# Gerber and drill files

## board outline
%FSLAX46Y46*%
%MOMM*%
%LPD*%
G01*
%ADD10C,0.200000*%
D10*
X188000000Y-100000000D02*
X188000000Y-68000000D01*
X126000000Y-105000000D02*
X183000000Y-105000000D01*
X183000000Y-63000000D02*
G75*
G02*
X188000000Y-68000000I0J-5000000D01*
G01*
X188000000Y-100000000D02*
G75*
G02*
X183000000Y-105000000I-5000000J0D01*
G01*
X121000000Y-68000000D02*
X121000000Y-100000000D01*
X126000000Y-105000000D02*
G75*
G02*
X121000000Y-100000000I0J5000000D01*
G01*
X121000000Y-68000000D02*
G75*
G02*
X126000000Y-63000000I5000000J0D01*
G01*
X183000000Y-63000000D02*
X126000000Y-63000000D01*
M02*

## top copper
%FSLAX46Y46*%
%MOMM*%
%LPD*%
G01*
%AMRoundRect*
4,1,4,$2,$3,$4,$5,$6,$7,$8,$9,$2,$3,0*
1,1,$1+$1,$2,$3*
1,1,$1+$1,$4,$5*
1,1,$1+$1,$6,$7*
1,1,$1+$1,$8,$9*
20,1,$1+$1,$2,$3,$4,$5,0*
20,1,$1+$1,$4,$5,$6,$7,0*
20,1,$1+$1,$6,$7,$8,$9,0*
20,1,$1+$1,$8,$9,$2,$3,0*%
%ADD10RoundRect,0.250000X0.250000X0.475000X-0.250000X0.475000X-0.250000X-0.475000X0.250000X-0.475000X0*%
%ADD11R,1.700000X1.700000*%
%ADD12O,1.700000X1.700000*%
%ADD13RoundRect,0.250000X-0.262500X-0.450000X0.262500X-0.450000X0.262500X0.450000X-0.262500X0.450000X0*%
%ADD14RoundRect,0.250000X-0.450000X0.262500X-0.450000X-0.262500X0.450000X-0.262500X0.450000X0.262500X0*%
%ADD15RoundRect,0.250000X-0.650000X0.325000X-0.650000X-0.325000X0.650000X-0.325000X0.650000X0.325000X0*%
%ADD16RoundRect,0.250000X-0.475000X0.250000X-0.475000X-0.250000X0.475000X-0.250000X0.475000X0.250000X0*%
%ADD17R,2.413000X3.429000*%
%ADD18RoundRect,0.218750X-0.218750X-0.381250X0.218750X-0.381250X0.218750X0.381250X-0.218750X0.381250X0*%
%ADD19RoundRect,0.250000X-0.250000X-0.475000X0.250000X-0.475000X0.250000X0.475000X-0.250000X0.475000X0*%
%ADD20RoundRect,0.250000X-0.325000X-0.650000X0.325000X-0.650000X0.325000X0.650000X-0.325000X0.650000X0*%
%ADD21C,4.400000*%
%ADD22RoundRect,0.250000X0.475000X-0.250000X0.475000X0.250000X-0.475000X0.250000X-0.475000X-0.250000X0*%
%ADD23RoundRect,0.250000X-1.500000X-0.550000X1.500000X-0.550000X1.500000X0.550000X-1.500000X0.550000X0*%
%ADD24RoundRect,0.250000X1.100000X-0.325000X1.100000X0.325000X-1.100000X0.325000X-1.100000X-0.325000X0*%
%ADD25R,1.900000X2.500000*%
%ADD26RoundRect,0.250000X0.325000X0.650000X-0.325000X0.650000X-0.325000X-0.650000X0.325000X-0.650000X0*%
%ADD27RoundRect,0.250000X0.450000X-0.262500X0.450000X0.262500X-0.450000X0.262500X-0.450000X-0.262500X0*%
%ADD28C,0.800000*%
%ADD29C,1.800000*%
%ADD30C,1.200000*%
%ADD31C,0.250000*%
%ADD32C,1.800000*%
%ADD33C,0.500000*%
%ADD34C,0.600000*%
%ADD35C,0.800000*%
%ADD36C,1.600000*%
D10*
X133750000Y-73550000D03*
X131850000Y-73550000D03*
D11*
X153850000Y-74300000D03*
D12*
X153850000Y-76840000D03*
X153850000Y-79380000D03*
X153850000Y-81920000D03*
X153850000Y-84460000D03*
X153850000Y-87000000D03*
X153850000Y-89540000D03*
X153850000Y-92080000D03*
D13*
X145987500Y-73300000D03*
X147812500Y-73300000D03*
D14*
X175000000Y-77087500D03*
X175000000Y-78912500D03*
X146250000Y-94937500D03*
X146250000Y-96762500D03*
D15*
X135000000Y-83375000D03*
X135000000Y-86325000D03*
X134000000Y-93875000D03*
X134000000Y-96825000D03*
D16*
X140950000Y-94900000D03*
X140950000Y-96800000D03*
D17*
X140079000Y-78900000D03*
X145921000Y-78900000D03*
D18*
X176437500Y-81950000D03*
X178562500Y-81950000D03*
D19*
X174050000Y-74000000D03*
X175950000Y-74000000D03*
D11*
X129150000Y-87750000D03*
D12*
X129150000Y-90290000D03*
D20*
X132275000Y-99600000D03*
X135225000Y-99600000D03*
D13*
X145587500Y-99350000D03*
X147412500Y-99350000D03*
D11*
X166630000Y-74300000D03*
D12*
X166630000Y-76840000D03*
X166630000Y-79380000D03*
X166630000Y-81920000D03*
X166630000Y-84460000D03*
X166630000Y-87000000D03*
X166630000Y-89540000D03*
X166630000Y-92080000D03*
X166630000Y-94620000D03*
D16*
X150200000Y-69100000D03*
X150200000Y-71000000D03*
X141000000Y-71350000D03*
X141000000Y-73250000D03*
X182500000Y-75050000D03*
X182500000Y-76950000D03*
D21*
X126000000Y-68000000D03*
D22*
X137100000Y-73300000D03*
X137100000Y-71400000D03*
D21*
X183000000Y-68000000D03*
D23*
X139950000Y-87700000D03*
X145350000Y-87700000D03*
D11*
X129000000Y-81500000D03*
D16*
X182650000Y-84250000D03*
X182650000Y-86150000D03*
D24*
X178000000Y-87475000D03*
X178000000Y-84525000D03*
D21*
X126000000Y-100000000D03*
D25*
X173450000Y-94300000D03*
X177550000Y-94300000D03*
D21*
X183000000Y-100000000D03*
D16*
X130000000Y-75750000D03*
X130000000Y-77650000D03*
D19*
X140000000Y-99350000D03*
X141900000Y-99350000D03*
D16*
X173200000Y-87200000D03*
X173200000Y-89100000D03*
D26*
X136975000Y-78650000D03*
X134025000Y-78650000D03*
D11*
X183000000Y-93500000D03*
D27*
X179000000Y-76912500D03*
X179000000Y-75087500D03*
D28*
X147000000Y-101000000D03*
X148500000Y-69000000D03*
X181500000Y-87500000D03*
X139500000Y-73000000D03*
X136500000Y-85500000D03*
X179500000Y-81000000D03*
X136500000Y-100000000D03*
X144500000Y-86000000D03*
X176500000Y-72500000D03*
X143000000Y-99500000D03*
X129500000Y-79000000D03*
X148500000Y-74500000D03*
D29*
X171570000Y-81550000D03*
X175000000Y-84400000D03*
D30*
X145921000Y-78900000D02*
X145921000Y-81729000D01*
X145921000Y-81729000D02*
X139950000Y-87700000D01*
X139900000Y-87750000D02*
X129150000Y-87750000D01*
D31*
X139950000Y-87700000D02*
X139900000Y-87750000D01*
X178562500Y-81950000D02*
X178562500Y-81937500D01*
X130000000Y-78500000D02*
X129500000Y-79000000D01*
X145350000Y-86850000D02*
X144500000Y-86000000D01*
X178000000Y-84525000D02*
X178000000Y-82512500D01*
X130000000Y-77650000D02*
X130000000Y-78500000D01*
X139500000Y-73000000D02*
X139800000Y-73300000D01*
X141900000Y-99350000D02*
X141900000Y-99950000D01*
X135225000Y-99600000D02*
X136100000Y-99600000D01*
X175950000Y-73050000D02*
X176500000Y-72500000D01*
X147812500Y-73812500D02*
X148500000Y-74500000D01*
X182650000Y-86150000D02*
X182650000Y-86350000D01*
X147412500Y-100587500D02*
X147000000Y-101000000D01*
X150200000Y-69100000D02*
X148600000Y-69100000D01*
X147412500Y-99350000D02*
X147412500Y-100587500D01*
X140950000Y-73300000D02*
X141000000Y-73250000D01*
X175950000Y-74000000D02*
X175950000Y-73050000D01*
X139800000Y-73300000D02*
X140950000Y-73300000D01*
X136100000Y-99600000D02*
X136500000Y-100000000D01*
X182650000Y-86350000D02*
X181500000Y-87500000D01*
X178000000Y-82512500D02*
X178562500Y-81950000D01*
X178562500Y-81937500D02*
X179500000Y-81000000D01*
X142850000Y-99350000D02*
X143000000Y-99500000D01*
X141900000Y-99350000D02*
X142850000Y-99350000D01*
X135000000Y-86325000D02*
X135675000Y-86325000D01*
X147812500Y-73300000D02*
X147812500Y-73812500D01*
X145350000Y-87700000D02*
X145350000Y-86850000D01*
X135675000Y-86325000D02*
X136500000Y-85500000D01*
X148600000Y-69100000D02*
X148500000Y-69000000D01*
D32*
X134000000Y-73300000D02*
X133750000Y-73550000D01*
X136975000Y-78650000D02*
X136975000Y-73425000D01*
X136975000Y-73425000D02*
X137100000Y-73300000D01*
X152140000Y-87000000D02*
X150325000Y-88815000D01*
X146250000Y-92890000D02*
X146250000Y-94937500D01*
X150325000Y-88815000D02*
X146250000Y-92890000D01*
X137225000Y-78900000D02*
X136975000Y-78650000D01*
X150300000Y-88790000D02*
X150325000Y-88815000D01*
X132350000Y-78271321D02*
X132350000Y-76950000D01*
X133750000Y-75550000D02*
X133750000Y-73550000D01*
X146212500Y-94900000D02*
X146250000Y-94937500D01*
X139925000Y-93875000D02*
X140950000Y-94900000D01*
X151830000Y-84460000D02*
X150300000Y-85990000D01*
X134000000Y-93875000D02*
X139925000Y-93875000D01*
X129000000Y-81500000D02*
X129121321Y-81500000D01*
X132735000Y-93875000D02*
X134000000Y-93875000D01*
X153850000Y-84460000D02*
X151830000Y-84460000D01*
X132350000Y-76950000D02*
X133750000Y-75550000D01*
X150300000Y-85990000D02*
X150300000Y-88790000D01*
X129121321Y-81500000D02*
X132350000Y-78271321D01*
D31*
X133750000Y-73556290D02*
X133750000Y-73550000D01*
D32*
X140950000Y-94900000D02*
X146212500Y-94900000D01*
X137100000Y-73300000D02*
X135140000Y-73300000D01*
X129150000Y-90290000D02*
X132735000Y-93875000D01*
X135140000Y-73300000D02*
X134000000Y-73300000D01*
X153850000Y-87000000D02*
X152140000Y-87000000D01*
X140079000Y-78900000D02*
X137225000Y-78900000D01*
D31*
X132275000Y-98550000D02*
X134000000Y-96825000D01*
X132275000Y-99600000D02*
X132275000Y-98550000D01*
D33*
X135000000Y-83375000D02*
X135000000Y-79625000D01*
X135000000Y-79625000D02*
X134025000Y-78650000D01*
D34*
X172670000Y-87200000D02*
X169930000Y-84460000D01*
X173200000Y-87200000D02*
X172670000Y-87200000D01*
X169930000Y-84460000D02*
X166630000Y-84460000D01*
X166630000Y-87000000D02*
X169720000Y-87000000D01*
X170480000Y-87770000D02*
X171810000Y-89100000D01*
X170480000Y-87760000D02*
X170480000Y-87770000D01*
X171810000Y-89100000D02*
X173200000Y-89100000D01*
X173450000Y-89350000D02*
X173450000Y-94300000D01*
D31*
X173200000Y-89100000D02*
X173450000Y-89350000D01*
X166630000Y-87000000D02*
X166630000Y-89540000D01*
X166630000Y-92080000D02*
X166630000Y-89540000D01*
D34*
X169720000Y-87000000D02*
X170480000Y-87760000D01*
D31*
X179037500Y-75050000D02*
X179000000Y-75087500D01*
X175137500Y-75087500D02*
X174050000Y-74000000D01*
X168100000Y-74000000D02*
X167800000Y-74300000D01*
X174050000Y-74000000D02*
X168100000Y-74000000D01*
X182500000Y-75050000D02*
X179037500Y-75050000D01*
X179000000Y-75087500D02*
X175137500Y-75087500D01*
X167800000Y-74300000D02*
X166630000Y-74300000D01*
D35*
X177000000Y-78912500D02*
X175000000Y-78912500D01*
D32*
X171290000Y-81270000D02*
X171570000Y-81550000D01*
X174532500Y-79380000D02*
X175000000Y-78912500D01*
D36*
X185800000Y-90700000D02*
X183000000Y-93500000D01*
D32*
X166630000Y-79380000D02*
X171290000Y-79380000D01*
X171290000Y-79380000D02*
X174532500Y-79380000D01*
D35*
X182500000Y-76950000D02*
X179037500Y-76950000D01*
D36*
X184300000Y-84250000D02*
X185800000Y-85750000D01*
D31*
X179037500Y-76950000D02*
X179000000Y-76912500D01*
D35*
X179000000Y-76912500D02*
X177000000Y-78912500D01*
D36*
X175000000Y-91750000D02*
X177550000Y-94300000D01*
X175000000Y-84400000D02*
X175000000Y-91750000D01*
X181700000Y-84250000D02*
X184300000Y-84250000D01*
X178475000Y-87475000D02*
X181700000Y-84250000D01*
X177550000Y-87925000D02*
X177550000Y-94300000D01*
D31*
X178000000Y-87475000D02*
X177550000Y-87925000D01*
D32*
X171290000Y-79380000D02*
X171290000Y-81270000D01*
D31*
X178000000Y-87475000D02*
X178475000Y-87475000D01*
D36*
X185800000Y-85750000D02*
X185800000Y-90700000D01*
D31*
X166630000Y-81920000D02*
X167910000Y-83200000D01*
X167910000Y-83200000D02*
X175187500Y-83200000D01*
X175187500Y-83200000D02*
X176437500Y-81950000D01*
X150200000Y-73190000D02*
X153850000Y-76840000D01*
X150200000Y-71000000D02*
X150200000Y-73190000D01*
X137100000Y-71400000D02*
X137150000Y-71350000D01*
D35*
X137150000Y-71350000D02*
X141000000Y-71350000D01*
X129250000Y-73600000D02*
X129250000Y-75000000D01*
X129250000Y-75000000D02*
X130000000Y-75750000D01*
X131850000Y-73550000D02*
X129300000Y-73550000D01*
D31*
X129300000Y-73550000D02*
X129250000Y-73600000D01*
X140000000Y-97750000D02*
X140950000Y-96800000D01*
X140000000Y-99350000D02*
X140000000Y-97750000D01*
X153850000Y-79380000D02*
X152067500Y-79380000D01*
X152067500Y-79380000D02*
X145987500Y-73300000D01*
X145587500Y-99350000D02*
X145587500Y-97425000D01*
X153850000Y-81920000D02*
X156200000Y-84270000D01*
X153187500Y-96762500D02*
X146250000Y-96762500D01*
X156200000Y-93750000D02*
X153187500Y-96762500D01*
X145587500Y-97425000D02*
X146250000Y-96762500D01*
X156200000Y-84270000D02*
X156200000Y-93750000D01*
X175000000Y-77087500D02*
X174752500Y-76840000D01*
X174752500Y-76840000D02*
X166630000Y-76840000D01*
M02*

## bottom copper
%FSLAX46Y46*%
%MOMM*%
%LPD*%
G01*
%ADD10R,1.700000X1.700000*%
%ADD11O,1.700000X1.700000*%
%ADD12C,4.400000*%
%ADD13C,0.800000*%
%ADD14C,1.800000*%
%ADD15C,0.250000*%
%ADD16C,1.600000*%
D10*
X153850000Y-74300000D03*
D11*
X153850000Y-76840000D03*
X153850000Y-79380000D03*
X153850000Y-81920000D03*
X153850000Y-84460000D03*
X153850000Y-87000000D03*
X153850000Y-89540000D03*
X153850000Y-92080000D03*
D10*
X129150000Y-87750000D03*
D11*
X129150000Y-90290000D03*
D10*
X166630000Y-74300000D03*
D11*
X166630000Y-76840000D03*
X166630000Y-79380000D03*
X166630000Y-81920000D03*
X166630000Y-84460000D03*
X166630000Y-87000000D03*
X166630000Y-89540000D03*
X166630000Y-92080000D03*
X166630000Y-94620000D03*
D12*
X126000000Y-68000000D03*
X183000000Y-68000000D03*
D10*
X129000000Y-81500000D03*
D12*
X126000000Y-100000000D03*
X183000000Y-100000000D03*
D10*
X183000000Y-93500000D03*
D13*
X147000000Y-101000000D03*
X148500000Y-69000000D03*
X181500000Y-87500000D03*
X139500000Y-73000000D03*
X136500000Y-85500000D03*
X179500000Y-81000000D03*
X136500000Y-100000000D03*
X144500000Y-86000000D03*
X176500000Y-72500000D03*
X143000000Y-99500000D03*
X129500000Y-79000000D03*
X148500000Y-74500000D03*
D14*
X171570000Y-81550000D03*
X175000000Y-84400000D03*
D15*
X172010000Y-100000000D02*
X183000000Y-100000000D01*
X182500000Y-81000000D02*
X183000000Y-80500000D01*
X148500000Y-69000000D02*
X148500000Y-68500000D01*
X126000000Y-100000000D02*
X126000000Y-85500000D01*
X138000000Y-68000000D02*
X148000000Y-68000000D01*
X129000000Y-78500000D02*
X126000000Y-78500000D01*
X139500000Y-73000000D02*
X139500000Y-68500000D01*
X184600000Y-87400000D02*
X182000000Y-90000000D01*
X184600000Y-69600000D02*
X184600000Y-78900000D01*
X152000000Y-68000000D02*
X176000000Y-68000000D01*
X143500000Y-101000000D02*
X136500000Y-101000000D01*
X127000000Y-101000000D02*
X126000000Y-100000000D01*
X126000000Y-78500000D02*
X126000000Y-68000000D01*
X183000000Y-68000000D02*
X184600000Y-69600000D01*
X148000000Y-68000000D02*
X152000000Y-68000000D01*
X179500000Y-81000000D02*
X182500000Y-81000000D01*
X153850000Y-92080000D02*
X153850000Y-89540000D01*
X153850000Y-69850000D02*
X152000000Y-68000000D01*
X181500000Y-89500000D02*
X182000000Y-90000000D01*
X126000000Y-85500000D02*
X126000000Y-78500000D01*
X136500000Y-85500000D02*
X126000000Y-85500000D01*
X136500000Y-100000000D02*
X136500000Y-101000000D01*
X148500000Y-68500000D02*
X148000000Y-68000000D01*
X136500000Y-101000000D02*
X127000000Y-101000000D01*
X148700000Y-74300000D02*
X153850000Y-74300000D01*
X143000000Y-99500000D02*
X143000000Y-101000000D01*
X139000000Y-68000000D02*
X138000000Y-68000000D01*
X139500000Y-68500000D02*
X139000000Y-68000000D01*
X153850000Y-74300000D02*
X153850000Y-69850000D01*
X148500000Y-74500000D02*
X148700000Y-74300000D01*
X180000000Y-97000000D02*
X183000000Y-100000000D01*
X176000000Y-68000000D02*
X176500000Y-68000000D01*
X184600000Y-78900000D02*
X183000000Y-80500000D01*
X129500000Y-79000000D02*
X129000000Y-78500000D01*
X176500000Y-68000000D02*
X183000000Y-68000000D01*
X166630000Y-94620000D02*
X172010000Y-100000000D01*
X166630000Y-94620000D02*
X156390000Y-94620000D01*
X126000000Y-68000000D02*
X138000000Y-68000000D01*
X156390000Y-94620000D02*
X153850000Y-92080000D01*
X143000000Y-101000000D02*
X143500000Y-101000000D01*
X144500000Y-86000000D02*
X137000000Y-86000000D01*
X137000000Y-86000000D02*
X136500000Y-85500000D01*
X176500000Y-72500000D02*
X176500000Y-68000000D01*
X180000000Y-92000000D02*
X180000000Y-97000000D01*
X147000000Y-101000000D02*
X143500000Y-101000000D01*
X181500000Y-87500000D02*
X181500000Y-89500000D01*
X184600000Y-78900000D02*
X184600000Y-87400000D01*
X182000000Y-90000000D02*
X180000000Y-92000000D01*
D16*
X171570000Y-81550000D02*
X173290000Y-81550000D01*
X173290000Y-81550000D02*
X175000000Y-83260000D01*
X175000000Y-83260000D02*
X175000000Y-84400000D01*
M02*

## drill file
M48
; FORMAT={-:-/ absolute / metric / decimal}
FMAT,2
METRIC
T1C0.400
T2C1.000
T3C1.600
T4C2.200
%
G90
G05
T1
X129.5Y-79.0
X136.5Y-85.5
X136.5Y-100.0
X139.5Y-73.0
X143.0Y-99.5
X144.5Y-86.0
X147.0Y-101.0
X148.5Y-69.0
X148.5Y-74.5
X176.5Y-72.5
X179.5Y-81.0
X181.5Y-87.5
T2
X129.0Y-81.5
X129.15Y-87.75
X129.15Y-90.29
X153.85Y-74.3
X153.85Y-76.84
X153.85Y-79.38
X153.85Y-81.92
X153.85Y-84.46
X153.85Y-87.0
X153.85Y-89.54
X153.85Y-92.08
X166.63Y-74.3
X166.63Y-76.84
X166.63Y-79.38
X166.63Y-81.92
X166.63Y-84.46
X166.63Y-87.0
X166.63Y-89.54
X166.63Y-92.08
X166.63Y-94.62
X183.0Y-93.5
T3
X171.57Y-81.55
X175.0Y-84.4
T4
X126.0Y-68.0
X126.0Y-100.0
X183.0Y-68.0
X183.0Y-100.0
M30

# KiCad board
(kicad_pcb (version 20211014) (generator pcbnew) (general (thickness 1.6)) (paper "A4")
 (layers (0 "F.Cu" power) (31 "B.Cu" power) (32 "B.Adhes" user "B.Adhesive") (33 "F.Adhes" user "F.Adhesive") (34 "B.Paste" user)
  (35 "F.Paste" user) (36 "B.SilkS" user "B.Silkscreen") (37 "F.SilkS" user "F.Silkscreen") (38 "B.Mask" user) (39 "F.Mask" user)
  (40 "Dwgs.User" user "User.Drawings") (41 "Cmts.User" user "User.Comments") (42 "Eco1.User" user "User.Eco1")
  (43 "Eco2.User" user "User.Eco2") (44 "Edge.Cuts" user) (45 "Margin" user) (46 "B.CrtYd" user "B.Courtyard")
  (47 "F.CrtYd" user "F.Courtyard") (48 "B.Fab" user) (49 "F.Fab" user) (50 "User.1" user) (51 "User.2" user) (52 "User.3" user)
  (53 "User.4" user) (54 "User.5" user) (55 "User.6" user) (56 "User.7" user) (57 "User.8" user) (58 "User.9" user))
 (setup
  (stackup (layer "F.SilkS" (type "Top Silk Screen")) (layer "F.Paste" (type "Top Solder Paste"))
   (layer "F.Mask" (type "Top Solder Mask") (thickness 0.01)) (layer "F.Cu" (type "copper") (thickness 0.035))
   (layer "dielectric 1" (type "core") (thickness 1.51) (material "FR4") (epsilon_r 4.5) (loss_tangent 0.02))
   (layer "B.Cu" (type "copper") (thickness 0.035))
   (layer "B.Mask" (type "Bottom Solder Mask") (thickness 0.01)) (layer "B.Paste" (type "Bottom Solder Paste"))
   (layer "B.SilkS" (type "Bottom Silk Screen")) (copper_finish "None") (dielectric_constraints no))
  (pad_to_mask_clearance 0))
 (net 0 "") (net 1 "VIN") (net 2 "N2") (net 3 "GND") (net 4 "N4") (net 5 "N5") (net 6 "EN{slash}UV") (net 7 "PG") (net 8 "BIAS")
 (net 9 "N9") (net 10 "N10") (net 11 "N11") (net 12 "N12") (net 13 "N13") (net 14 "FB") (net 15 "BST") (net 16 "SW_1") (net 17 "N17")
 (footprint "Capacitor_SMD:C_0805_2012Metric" (layer "F.Cu") (at 132.8 73.55 180)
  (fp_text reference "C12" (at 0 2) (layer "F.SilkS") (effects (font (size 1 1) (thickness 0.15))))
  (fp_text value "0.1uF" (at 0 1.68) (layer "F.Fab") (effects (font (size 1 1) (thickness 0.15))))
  (pad "1" smd roundrect (at -0.95 0 180) (size 1 1.45) (layers "F.Cu" "F.Paste" "F.Mask") (roundrect_rratio 0.25) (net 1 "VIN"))
  (pad "2" smd roundrect (at 0.95 0 180) (size 1 1.45) (layers "F.Cu" "F.Paste" "F.Mask") (roundrect_rratio 0.25) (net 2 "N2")))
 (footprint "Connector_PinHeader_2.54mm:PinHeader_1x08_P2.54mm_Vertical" (layer "F.Cu") (at 153.85 74.3)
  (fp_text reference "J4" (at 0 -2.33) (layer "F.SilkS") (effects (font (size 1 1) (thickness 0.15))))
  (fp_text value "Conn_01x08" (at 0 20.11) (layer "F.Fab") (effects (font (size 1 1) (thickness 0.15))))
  (pad "1" thru_hole rect (at 0 0) (size 1.7 1.7) (drill 1) (layers *.Cu *.Mask) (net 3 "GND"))
  (pad "2" thru_hole oval (at 0 2.54) (size 1.7 1.7) (drill 1) (layers *.Cu *.Mask) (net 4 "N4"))
  (pad "3" thru_hole oval (at 0 5.08) (size 1.7 1.7) (drill 1) (layers *.Cu *.Mask) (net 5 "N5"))
  (pad "4" thru_hole oval (at 0 7.62) (size 1.7 1.7) (drill 1) (layers *.Cu *.Mask) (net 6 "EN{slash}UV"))
  (pad "5" thru_hole oval (at 0 10.16) (size 1.7 1.7) (drill 1) (layers *.Cu *.Mask) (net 1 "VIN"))
  (pad "6" thru_hole oval (at 0 12.7) (size 1.7 1.7) (drill 1) (layers *.Cu *.Mask) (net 1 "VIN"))
  (pad "7" thru_hole oval (at 0 15.24) (size 1.7 1.7) (drill 1) (layers *.Cu *.Mask) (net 3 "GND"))
  (pad "8" thru_hole oval (at 0 17.78) (size 1.7 1.7) (drill 1) (layers *.Cu *.Mask) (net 3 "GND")))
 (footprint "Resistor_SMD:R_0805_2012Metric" (layer "F.Cu") (at 146.9 73.3)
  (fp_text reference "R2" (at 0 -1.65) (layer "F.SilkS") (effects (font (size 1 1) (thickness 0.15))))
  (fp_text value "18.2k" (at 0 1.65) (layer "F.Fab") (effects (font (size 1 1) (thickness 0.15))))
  (pad "1" smd roundrect (at -0.9125 0) (size 1.025 1.4) (layers "F.Cu" "F.Paste" "F.Mask") (roundrect_rratio 0.243902) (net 5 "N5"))
  (pad "2" smd roundrect (at 0.9125 0) (size 1.025 1.4) (layers "F.Cu" "F.Paste" "F.Mask") (roundrect_rratio 0.243902) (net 3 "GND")))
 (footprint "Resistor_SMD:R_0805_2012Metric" (layer "F.Cu") (at 175 78 -90)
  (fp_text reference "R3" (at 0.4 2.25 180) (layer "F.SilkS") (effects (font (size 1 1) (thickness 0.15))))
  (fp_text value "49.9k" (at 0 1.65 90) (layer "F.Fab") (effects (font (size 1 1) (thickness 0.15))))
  (pad "1" smd roundrect (at -0.9125 0 270) (size 1.025 1.4) (layers "F.Cu" "F.Paste" "F.Mask") (roundrect_rratio 0.243902) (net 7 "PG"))
  (pad "2" smd roundrect (at 0.9125 0 270) (size 1.025 1.4) (layers "F.Cu" "F.Paste" "F.Mask") (roundrect_rratio 0.243902) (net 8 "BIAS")))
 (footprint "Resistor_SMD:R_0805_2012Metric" (layer "F.Cu") (at 146.25 95.85 -90)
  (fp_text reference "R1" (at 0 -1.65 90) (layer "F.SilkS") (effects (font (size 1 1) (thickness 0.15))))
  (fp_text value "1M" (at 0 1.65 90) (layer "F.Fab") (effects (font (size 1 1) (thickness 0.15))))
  (pad "1" smd roundrect (at -0.9125 0 270) (size 1.025 1.4) (layers "F.Cu" "F.Paste" "F.Mask") (roundrect_rratio 0.243902) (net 1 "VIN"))
  (pad "2" smd roundrect (at 0.9125 0 270) (size 1.025 1.4) (layers "F.Cu" "F.Paste" "F.Mask") (roundrect_rratio 0.243902)
   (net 6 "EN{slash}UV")))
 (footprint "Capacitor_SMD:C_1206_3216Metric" (layer "F.Cu") (at 135 84.85 -90)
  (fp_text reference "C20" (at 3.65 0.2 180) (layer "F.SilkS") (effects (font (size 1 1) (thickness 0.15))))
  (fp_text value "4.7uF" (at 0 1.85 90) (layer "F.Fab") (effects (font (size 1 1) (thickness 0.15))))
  (pad "1" smd roundrect (at -1.475 0 270) (size 1.15 1.8) (layers "F.Cu" "F.Paste" "F.Mask") (roundrect_rratio 0.217391) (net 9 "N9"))
  (pad "2" smd roundrect (at 1.475 0 270) (size 1.15 1.8) (layers "F.Cu" "F.Paste" "F.Mask") (roundrect_rratio 0.217391) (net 3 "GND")))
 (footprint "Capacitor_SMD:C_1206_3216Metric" (layer "F.Cu") (at 134 95.35 -90)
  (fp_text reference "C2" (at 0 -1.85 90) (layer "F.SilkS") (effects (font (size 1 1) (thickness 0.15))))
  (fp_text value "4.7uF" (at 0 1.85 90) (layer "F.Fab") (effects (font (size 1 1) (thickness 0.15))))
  (pad "1" smd roundrect (at -1.475 0 270) (size 1.15 1.8) (layers "F.Cu" "F.Paste" "F.Mask") (roundrect_rratio 0.217391) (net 1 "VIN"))
  (pad "2" smd roundrect (at 1.475 0 270) (size 1.15 1.8) (layers "F.Cu" "F.Paste" "F.Mask") (roundrect_rratio 0.217391) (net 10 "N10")))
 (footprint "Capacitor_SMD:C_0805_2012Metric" (layer "F.Cu") (at 140.95 95.85 -90)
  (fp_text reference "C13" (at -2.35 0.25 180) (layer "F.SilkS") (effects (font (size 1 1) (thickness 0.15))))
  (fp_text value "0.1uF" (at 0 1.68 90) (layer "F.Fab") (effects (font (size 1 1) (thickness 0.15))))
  (pad "1" smd roundrect (at -0.95 0 270) (size 1 1.45) (layers "F.Cu" "F.Paste" "F.Mask") (roundrect_rratio 0.25) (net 1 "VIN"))
  (pad "2" smd roundrect (at 0.95 0 270) (size 1 1.45) (layers "F.Cu" "F.Paste" "F.Mask") (roundrect_rratio 0.25) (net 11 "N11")))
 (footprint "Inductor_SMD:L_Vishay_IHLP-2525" (layer "F.Cu") (at 143 78.9)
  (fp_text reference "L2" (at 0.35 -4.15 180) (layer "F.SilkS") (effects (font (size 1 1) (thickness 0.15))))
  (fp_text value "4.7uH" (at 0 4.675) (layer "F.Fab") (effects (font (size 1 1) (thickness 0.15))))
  (pad "1" smd rect (at -2.921 0) (size 2.413 3.429) (layers "F.Cu" "F.Paste" "F.Mask") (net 1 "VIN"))
  (pad "2" smd rect (at 2.921 0) (size 2.413 3.429) (layers "F.Cu" "F.Paste" "F.Mask") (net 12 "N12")))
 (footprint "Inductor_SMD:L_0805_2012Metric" (layer "F.Cu") (at 177.5 81.95)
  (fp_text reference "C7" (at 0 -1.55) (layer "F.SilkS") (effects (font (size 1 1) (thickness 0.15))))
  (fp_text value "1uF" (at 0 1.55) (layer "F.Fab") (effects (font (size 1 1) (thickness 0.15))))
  (pad "1" smd roundrect (at -1.0625 0) (size 0.875 1.2) (layers "F.Cu" "F.Paste" "F.Mask") (roundrect_rratio 0.25) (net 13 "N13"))
  (pad "2" smd roundrect (at 1.0625 0) (size 0.875 1.2) (layers "F.Cu" "F.Paste" "F.Mask") (roundrect_rratio 0.25) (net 3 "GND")))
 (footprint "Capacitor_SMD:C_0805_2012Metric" (layer "F.Cu") (at 175 74)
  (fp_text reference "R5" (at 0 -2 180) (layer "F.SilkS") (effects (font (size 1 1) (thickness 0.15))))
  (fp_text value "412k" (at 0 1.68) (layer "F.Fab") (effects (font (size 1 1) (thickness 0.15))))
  (pad "1" smd roundrect (at -0.95 0) (size 1 1.45) (layers "F.Cu" "F.Paste" "F.Mask") (roundrect_rratio 0.25) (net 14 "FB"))
  (pad "2" smd roundrect (at 0.95 0) (size 1 1.45) (layers "F.Cu" "F.Paste" "F.Mask") (roundrect_rratio 0.25) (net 3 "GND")))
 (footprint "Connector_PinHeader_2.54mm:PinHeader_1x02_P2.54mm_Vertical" (layer "F.Cu") (at 129.15 87.75)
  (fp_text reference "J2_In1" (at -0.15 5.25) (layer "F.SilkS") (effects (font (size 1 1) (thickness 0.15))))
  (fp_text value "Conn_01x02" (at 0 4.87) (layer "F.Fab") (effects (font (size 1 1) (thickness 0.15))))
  (pad "1" thru_hole rect (at 0 0) (size 1.7 1.7) (drill 1) (layers *.Cu *.Mask) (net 12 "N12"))
  (pad "2" thru_hole oval (at 0 2.54) (size 1.7 1.7) (drill 1) (layers *.Cu *.Mask) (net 1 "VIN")))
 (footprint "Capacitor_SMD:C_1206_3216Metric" (layer "F.Cu") (at 133.75 99.6)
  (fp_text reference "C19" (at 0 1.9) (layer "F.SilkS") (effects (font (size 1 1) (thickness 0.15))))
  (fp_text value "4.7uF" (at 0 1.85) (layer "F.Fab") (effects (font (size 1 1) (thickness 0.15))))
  (pad "1" smd roundrect (at -1.475 0) (size 1.15 1.8) (layers "F.Cu" "F.Paste" "F.Mask") (roundrect_rratio 0.217391) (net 10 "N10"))
  (pad "2" smd roundrect (at 1.475 0) (size 1.15 1.8) (layers "F.Cu" "F.Paste" "F.Mask") (roundrect_rratio 0.217391) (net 3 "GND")))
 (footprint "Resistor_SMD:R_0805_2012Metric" (layer "F.Cu") (at 146.5 99.35)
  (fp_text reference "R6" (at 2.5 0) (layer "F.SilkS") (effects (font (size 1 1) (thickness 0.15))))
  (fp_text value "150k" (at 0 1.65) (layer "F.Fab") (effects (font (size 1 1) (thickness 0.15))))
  (pad "1" smd roundrect (at -0.9125 0) (size 1.025 1.4) (layers "F.Cu" "F.Paste" "F.Mask") (roundrect_rratio 0.243902)
   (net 6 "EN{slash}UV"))
  (pad "2" smd roundrect (at 0.9125 0) (size 1.025 1.4) (layers "F.Cu" "F.Paste" "F.Mask") (roundrect_rratio 0.243902) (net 3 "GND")))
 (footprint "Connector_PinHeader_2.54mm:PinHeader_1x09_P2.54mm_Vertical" (layer "F.Cu") (at 166.63 74.3)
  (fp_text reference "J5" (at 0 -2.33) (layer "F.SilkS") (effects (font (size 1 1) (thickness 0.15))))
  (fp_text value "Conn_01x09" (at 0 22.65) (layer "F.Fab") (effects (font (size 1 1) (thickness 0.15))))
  (pad "1" thru_hole rect (at 0 0) (size 1.7 1.7) (drill 1) (layers *.Cu *.Mask) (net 14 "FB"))
  (pad "2" thru_hole oval (at 0 2.54) (size 1.7 1.7) (drill 1) (layers *.Cu *.Mask) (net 7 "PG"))
  (pad "3" thru_hole oval (at 0 5.08) (size 1.7 1.7) (drill 1) (layers *.Cu *.Mask) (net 8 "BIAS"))
  (pad "4" thru_hole oval (at 0 7.62) (size 1.7 1.7) (drill 1) (layers *.Cu *.Mask) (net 13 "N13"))
  (pad "5" thru_hole oval (at 0 10.16) (size 1.7 1.7) (drill 1) (layers *.Cu *.Mask) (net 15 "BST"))
  (pad "6" thru_hole oval (at 0 12.7) (size 1.7 1.7) (drill 1) (layers *.Cu *.Mask) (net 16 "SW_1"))
  (pad "7" thru_hole oval (at 0 15.24) (size 1.7 1.7) (drill 1) (layers *.Cu *.Mask) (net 16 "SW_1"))
  (pad "8" thru_hole oval (at 0 17.78) (size 1.7 1.7) (drill 1) (layers *.Cu *.Mask) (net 16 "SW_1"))
  (pad "9" thru_hole oval (at 0 20.32) (size 1.7 1.7) (drill 1) (layers *.Cu *.Mask) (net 3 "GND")))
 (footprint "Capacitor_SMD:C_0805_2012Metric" (layer "F.Cu") (at 150.2 70.05 -90)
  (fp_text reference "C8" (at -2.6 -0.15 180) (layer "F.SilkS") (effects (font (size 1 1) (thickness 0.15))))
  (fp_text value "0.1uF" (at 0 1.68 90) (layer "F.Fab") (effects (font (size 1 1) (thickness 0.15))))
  (pad "1" smd roundrect (at -0.95 0 270) (size 1 1.45) (layers "F.Cu" "F.Paste" "F.Mask") (roundrect_rratio 0.25) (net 3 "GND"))
  (pad "2" smd roundrect (at 0.95 0 270) (size 1 1.45) (layers "F.Cu" "F.Paste" "F.Mask") (roundrect_rratio 0.25) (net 4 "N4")))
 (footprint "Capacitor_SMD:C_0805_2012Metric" (layer "F.Cu") (at 141 72.3 -90)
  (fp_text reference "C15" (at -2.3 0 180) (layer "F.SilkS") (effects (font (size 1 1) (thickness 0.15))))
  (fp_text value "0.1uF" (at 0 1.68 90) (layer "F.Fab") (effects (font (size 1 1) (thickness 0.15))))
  (pad "1" smd roundrect (at -0.95 0 270) (size 1 1.45) (layers "F.Cu" "F.Paste" "F.Mask") (roundrect_rratio 0.25) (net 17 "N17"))
  (pad "2" smd roundrect (at 0.95 0 270) (size 1 1.45) (layers "F.Cu" "F.Paste" "F.Mask") (roundrect_rratio 0.25) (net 3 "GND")))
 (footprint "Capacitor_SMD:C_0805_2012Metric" (layer "F.Cu") (at 182.5 76 -90)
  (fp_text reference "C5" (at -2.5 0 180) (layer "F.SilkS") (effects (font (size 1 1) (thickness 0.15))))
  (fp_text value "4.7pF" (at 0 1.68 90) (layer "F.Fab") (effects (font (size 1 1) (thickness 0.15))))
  (pad "1" smd roundrect (at -0.95 0 270) (size 1 1.45) (layers "F.Cu" "F.Paste" "F.Mask") (roundrect_rratio 0.25) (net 14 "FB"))
  (pad "2" smd roundrect (at 0.95 0 270) (size 1 1.45) (layers "F.Cu" "F.Paste" "F.Mask") (roundrect_rratio 0.25) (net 8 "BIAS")))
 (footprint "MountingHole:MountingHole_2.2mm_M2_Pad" (layer "F.Cu") (at 126 68)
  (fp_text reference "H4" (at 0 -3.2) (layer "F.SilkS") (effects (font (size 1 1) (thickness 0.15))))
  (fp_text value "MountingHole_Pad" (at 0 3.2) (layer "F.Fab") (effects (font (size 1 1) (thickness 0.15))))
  (pad "1" thru_hole circle (at 0 0) (size 4.4 4.4) (drill 2.2) (layers *.Cu *.Mask) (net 3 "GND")))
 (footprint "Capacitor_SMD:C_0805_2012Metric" (layer "F.Cu") (at 137.1 72.35 90)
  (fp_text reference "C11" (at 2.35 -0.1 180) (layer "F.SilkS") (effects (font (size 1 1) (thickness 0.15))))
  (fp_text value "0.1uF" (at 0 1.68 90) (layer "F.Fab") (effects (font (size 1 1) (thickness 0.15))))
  (pad "1" smd roundrect (at -0.95 0 90) (size 1 1.45) (layers "F.Cu" "F.Paste" "F.Mask") (roundrect_rratio 0.25) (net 1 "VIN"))
  (pad "2" smd roundrect (at 0.95 0 90) (size 1 1.45) (layers "F.Cu" "F.Paste" "F.Mask") (roundrect_rratio 0.25) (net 17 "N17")))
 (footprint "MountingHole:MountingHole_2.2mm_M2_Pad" (layer "F.Cu") (at 183 68)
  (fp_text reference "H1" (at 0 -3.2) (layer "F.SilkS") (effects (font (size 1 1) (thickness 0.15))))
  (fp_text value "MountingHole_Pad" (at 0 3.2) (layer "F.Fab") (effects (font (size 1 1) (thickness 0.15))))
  (pad "1" thru_hole circle (at 0 0) (size 4.4 4.4) (drill 2.2) (layers *.Cu *.Mask) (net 3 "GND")))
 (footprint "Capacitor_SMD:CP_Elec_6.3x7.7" (layer "F.Cu") (at 142.65 87.7)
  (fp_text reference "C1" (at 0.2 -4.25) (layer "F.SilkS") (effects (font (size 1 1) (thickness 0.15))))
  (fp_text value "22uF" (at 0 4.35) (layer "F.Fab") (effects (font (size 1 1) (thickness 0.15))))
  (pad "1" smd roundrect (at -2.7 0) (size 3.5 1.6) (layers "F.Cu" "F.Paste" "F.Mask") (roundrect_rratio 0.15625) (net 12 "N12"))
  (pad "2" smd roundrect (at 2.7 0) (size 3.5 1.6) (layers "F.Cu" "F.Paste" "F.Mask") (roundrect_rratio 0.15625) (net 3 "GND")))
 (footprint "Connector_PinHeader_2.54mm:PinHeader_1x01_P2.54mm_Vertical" (layer "F.Cu") (at 129 81.5)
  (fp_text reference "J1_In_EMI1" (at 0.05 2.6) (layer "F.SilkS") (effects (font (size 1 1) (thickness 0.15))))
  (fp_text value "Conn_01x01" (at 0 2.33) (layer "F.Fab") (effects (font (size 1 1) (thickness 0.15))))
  (pad "1" thru_hole rect (at 0 0) (size 1.7 1.7) (drill 1) (layers *.Cu *.Mask) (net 1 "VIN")))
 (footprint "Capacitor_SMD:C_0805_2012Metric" (layer "F.Cu") (at 182.65 85.2 -90)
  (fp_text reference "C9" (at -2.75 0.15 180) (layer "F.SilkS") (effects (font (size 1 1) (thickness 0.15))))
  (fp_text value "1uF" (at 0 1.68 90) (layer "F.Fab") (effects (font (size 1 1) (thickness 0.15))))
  (pad "1" smd roundrect (at -0.95 0 270) (size 1 1.45) (layers "F.Cu" "F.Paste" "F.Mask") (roundrect_rratio 0.25) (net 8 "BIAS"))
  (pad "2" smd roundrect (at 0.95 0 270) (size 1 1.45) (layers "F.Cu" "F.Paste" "F.Mask") (roundrect_rratio 0.25) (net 3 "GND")))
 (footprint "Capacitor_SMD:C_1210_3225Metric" (layer "F.Cu") (at 178 86 90)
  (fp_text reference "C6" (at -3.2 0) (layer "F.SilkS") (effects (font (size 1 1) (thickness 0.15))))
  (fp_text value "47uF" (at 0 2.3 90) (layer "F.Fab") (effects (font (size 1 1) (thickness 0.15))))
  (pad "1" smd roundrect (at -1.475 0 90) (size 1.15 2.7) (layers "F.Cu" "F.Paste" "F.Mask") (roundrect_rratio 0.217391) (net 8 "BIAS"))
  (pad "2" smd roundrect (at 1.475 0 90) (size 1.15 2.7) (layers "F.Cu" "F.Paste" "F.Mask") (roundrect_rratio 0.217391) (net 3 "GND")))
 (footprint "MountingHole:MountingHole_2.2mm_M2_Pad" (layer "F.Cu") (at 126 100)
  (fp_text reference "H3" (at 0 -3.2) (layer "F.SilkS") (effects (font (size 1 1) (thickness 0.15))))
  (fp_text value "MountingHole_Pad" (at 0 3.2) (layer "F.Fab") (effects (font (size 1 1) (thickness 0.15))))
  (pad "1" thru_hole circle (at 0 0) (size 4.4 4.4) (drill 2.2) (layers *.Cu *.Mask) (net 3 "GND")))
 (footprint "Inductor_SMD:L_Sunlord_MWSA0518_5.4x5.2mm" (layer "F.Cu") (at 175.5 94.3)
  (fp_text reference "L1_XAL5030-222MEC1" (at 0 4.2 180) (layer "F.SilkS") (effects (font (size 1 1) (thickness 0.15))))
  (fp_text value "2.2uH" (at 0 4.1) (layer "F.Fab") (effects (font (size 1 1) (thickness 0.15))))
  (pad "1" smd rect (at -2.05 0) (size 1.9 2.5) (layers "F.Cu" "F.Paste" "F.Mask") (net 16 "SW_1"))
  (pad "2" smd rect (at 2.05 0) (size 1.9 2.5) (layers "F.Cu" "F.Paste" "F.Mask") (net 8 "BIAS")))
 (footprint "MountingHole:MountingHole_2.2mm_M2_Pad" (layer "F.Cu") (at 183 100)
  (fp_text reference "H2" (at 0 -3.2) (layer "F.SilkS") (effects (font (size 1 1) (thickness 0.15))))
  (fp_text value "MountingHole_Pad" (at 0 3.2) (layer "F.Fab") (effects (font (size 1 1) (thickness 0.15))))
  (pad "1" thru_hole circle (at 0 0) (size 4.4 4.4) (drill 2.2) (layers *.Cu *.Mask) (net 3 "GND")))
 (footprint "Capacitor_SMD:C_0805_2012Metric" (layer "F.Cu") (at 130 76.7 -90)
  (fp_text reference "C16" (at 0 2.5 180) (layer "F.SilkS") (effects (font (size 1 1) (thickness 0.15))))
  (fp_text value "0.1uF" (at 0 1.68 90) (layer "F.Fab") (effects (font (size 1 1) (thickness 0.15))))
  (pad "1" smd roundrect (at -0.95 0 270) (size 1 1.45) (layers "F.Cu" "F.Paste" "F.Mask") (roundrect_rratio 0.25) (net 2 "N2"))
  (pad "2" smd roundrect (at 0.95 0 270) (size 1 1.45) (layers "F.Cu" "F.Paste" "F.Mask") (roundrect_rratio 0.25) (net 3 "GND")))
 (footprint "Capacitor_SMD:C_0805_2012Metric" (layer "F.Cu") (at 140.95 99.35)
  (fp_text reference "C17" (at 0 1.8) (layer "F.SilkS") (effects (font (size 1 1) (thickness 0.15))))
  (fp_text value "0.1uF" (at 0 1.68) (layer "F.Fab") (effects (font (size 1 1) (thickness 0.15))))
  (pad "1" smd roundrect (at -0.95 0) (size 1 1.45) (layers "F.Cu" "F.Paste" "F.Mask") (roundrect_rratio 0.25) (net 11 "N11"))
  (pad "2" smd roundrect (at 0.95 0) (size 1 1.45) (layers "F.Cu" "F.Paste" "F.Mask") (roundrect_rratio 0.25) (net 3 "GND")))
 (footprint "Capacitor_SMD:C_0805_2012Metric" (layer "F.Cu") (at 173.2 88.15 -90)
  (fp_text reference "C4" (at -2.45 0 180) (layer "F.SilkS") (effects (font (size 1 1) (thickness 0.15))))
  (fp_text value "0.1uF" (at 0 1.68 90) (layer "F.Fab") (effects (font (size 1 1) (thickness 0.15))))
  (pad "1" smd roundrect (at -0.95 0 270) (size 1 1.45) (layers "F.Cu" "F.Paste" "F.Mask") (roundrect_rratio 0.25) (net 15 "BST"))
  (pad "2" smd roundrect (at 0.95 0 270) (size 1 1.45) (layers "F.Cu" "F.Paste" "F.Mask") (roundrect_rratio 0.25) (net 16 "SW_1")))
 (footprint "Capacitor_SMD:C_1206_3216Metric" (layer "F.Cu") (at 135.5 78.65 180)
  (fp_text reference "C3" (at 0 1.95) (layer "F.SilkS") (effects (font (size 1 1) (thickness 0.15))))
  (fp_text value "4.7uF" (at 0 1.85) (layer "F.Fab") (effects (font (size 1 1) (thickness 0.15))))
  (pad "1" smd roundrect (at -1.475 0 180) (size 1.15 1.8) (layers "F.Cu" "F.Paste" "F.Mask") (roundrect_rratio 0.217391) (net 1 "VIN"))
  (pad "2" smd roundrect (at 1.475 0 180) (size 1.15 1.8) (layers "F.Cu" "F.Paste" "F.Mask") (roundrect_rratio 0.217391) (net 9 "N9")))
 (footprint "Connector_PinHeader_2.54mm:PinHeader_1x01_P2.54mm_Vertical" (layer "F.Cu") (at 183 93.5)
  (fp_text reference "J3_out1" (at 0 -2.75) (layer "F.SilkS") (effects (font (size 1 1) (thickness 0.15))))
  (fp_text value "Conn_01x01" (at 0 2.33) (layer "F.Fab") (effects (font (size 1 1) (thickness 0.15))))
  (pad "1" thru_hole rect (at 0 0) (size 1.7 1.7) (drill 1) (layers *.Cu *.Mask) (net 8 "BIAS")))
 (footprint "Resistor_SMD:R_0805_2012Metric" (layer "F.Cu") (at 179 76 90)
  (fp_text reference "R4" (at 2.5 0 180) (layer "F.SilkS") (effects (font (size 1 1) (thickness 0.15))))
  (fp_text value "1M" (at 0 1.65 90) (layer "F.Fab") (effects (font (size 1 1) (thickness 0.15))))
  (pad "1" smd roundrect (at -0.9125 0 90) (size 1.025 1.4) (layers "F.Cu" "F.Paste" "F.Mask") (roundrect_rratio 0.243902) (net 8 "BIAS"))
  (pad "2" smd roundrect (at 0.9125 0 90) (size 1.025 1.4) (layers "F.Cu" "F.Paste" "F.Mask") (roundrect_rratio 0.243902) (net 14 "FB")))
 (gr_line (start 188 100) (end 188 68) (layer "Edge.Cuts") (width 0.2))
 (gr_line (start 126 105) (end 183 105) (layer "Edge.Cuts") (width 0.2))
 (gr_arc (start 183 63) (mid 186.535534 64.464466) (end 188 68) (layer "Edge.Cuts") (width 0.2))
 (gr_arc (start 188 100) (mid 186.535534 103.535534) (end 183 105) (layer "Edge.Cuts") (width 0.2))
 (gr_line (start 121 68) (end 121 100) (layer "Edge.Cuts") (width 0.2))
 (gr_arc (start 126 105) (mid 122.464466 103.535534) (end 121 100) (layer "Edge.Cuts") (width 0.2))
 (gr_arc (start 121 68) (mid 122.464466 64.464466) (end 126 63) (layer "Edge.Cuts") (width 0.2))
 (gr_line (start 183 63) (end 126 63) (layer "Edge.Cuts") (width 0.2))
 (segment (start 145.921 78.9) (end 145.921 81.729) (width 1.2) (layer "F.Cu") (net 12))
 (segment (start 145.921 81.729) (end 139.95 87.7) (width 1.2) (layer "F.Cu") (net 12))
 (segment (start 139.9 87.75) (end 129.15 87.75) (width 1.2) (layer "F.Cu") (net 12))
 (segment (start 139.95 87.7) (end 139.9 87.75) (width 0.25) (layer "F.Cu") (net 12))
 (segment (start 178.5625 81.95) (end 178.5625 81.9375) (width 0.25) (layer "F.Cu") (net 3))
 (segment (start 130 78.5) (end 129.5 79) (width 0.25) (layer "F.Cu") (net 3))
 (segment (start 145.35 86.85) (end 144.5 86) (width 0.25) (layer "F.Cu") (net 3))
 (segment (start 178 84.525) (end 178 82.5125) (width 0.25) (layer "F.Cu") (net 3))
 (segment (start 130 77.65) (end 130 78.5) (width 0.25) (layer "F.Cu") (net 3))
 (segment (start 139.5 73) (end 139.8 73.3) (width 0.25) (layer "F.Cu") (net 3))
 (segment (start 141.9 99.35) (end 141.9 99.95) (width 0.25) (layer "F.Cu") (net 3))
 (segment (start 135.225 99.6) (end 136.1 99.6) (width 0.25) (layer "F.Cu") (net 3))
 (segment (start 175.95 73.05) (end 176.5 72.5) (width 0.25) (layer "F.Cu") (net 3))
 (segment (start 147.8125 73.8125) (end 148.5 74.5) (width 0.25) (layer "F.Cu") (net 3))
 (segment (start 182.65 86.15) (end 182.65 86.35) (width 0.25) (layer "F.Cu") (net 3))
 (segment (start 147.4125 100.5875) (end 147 101) (width 0.25) (layer "F.Cu") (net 3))
 (segment (start 150.2 69.1) (end 148.6 69.1) (width 0.25) (layer "F.Cu") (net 3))
 (segment (start 147.4125 99.35) (end 147.4125 100.5875) (width 0.25) (layer "F.Cu") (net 3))
 (segment (start 140.95 73.3) (end 141 73.25) (width 0.25) (layer "F.Cu") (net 3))
 (segment (start 175.95 74) (end 175.95 73.05) (width 0.25) (layer "F.Cu") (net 3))
 (segment (start 139.8 73.3) (end 140.95 73.3) (width 0.25) (layer "F.Cu") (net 3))
 (segment (start 136.1 99.6) (end 136.5 100) (width 0.25) (layer "F.Cu") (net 3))
 (segment (start 182.65 86.35) (end 181.5 87.5) (width 0.25) (layer "F.Cu") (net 3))
 (segment (start 178 82.5125) (end 178.5625 81.95) (width 0.25) (layer "F.Cu") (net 3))
 (segment (start 178.5625 81.9375) (end 179.5 81) (width 0.25) (layer "F.Cu") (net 3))
 (segment (start 142.85 99.35) (end 143 99.5) (width 0.25) (layer "F.Cu") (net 3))
 (segment (start 141.9 99.35) (end 142.85 99.35) (width 0.25) (layer "F.Cu") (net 3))
 (segment (start 135 86.325) (end 135.675 86.325) (width 0.25) (layer "F.Cu") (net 3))
 (segment (start 147.8125 73.3) (end 147.8125 73.8125) (width 0.25) (layer "F.Cu") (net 3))
 (segment (start 145.35 87.7) (end 145.35 86.85) (width 0.25) (layer "F.Cu") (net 3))
 (segment (start 135.675 86.325) (end 136.5 85.5) (width 0.25) (layer "F.Cu") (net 3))
 (segment (start 148.6 69.1) (end 148.5 69) (width 0.25) (layer "F.Cu") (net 3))
 (via (at 147 101) (size 0.8) (drill 0.4) (layers "F.Cu" "B.Cu") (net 3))
 (via (at 148.5 69) (size 0.8) (drill 0.4) (layers "F.Cu" "B.Cu") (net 3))
 (via (at 181.5 87.5) (size 0.8) (drill 0.4) (layers "F.Cu" "B.Cu") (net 3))
 (via (at 139.5 73) (size 0.8) (drill 0.4) (layers "F.Cu" "B.Cu") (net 3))
 (via (at 136.5 85.5) (size 0.8) (drill 0.4) (layers "F.Cu" "B.Cu") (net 3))
 (via (at 179.5 81) (size 0.8) (drill 0.4) (layers "F.Cu" "B.Cu") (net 3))
 (via (at 136.5 100) (size 0.8) (drill 0.4) (layers "F.Cu" "B.Cu") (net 3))
 (via (at 144.5 86) (size 0.8) (drill 0.4) (layers "F.Cu" "B.Cu") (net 3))
 (via (at 176.5 72.5) (size 0.8) (drill 0.4) (layers "F.Cu" "B.Cu") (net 3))
 (via (at 143 99.5) (size 0.8) (drill 0.4) (layers "F.Cu" "B.Cu") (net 3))
 (via (at 129.5 79) (size 0.8) (drill 0.4) (layers "F.Cu" "B.Cu") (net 3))
 (via (at 148.5 74.5) (size 0.8) (drill 0.4) (layers "F.Cu" "B.Cu") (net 3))
 (segment (start 172.01 100) (end 183 100) (width 0.25) (layer "B.Cu") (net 3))
 (segment (start 182.5 81) (end 183 80.5) (width 0.25) (layer "B.Cu") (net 3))
 (segment (start 148.5 69) (end 148.5 68.5) (width 0.25) (layer "B.Cu") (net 3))
 (segment (start 126 100) (end 126 85.5) (width 0.25) (layer "B.Cu") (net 3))
 (segment (start 138 68) (end 148 68) (width 0.25) (layer "B.Cu") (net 3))
 (segment (start 129 78.5) (end 126 78.5) (width 0.25) (layer "B.Cu") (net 3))
 (segment (start 139.5 73) (end 139.5 68.5) (width 0.25) (layer "B.Cu") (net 3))
 (segment (start 184.6 87.4) (end 182 90) (width 0.25) (layer "B.Cu") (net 3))
 (segment (start 184.6 69.6) (end 184.6 78.9) (width 0.25) (layer "B.Cu") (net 3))
 (segment (start 152 68) (end 176 68) (width 0.25) (layer "B.Cu") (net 3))
 (segment (start 143.5 101) (end 136.5 101) (width 0.25) (layer "B.Cu") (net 3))
 (segment (start 127 101) (end 126 100) (width 0.25) (layer "B.Cu") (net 3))
 (segment (start 126 78.5) (end 126 68) (width 0.25) (layer "B.Cu") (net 3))
 (segment (start 183 68) (end 184.6 69.6) (width 0.25) (layer "B.Cu") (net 3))
 (segment (start 148 68) (end 152 68) (width 0.25) (layer "B.Cu") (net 3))
 (segment (start 179.5 81) (end 182.5 81) (width 0.25) (layer "B.Cu") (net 3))
 (segment (start 153.85 92.08) (end 153.85 89.54) (width 0.25) (layer "B.Cu") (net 3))
 (segment (start 153.85 69.85) (end 152 68) (width 0.25) (layer "B.Cu") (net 3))
 (segment (start 181.5 89.5) (end 182 90) (width 0.25) (layer "B.Cu") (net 3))
 (segment (start 126 85.5) (end 126 78.5) (width 0.25) (layer "B.Cu") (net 3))
 (segment (start 136.5 85.5) (end 126 85.5) (width 0.25) (layer "B.Cu") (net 3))
 (segment (start 136.5 100) (end 136.5 101) (width 0.25) (layer "B.Cu") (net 3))
 (segment (start 148.5 68.5) (end 148 68) (width 0.25) (layer "B.Cu") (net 3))
 (segment (start 136.5 101) (end 127 101) (width 0.25) (layer "B.Cu") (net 3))
 (segment (start 148.7 74.3) (end 153.85 74.3) (width 0.25) (layer "B.Cu") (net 3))
 (segment (start 143 99.5) (end 143 101) (width 0.25) (layer "B.Cu") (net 3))
 (segment (start 139 68) (end 138 68) (width 0.25) (layer "B.Cu") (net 3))
 (segment (start 139.5 68.5) (end 139 68) (width 0.25) (layer "B.Cu") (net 3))
 (segment (start 153.85 74.3) (end 153.85 69.85) (width 0.25) (layer "B.Cu") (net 3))
 (segment (start 148.5 74.5) (end 148.7 74.3) (width 0.25) (layer "B.Cu") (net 3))
 (segment (start 180 97) (end 183 100) (width 0.25) (layer "B.Cu") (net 3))
 (segment (start 176 68) (end 176.5 68) (width 0.25) (layer "B.Cu") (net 3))
 (segment (start 184.6 78.9) (end 183 80.5) (width 0.25) (layer "B.Cu") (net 3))
 (segment (start 129.5 79) (end 129 78.5) (width 0.25) (layer "B.Cu") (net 3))
 (segment (start 176.5 68) (end 183 68) (width 0.25) (layer "B.Cu") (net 3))
 (segment (start 166.63 94.62) (end 172.01 100) (width 0.25) (layer "B.Cu") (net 3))
 (segment (start 166.63 94.62) (end 156.39 94.62) (width 0.25) (layer "B.Cu") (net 3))
 (segment (start 126 68) (end 138 68) (width 0.25) (layer "B.Cu") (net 3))
 (segment (start 156.39 94.62) (end 153.85 92.08) (width 0.25) (layer "B.Cu") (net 3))
 (segment (start 143 101) (end 143.5 101) (width 0.25) (layer "B.Cu") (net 3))
 (segment (start 144.5 86) (end 137 86) (width 0.25) (layer "B.Cu") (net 3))
 (segment (start 137 86) (end 136.5 85.5) (width 0.25) (layer "B.Cu") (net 3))
 (segment (start 176.5 72.5) (end 176.5 68) (width 0.25) (layer "B.Cu") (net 3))
 (segment (start 180 92) (end 180 97) (width 0.25) (layer "B.Cu") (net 3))
 (segment (start 147 101) (end 143.5 101) (width 0.25) (layer "B.Cu") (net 3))
 (segment (start 181.5 87.5) (end 181.5 89.5) (width 0.25) (layer "B.Cu") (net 3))
 (segment (start 184.6 78.9) (end 184.6 87.4) (width 0.25) (layer "B.Cu") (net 3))
 (segment (start 182 90) (end 180 92) (width 0.25) (layer "B.Cu") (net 3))
 (segment (start 134 73.3) (end 133.75 73.55) (width 1.8) (layer "F.Cu") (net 1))
 (segment (start 136.975 78.65) (end 136.975 73.425) (width 1.8) (layer "F.Cu") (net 1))
 (segment (start 136.975 73.425) (end 137.1 73.3) (width 1.8) (layer "F.Cu") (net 1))
 (segment (start 152.14 87) (end 150.325 88.815) (width 1.8) (layer "F.Cu") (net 1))
 (segment (start 146.25 92.89) (end 146.25 94.9375) (width 1.8) (layer "F.Cu") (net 1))
 (segment (start 150.325 88.815) (end 146.25 92.89) (width 1.8) (layer "F.Cu") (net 1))
 (segment (start 137.225 78.9) (end 136.975 78.65) (width 1.8) (layer "F.Cu") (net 1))
 (segment (start 150.3 88.79) (end 150.325 88.815) (width 1.8) (layer "F.Cu") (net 1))
 (segment (start 132.35 78.271321) (end 132.35 76.95) (width 1.8) (layer "F.Cu") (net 1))
 (segment (start 133.75 75.55) (end 133.75 73.55) (width 1.8) (layer "F.Cu") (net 1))
 (segment (start 146.2125 94.9) (end 146.25 94.9375) (width 1.8) (layer "F.Cu") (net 1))
 (segment (start 139.925 93.875) (end 140.95 94.9) (width 1.8) (layer "F.Cu") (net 1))
 (segment (start 151.83 84.46) (end 150.3 85.99) (width 1.8) (layer "F.Cu") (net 1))
 (segment (start 134 93.875) (end 139.925 93.875) (width 1.8) (layer "F.Cu") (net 1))
 (segment (start 129 81.5) (end 129.121321 81.5) (width 1.8) (layer "F.Cu") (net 1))
 (segment (start 132.735 93.875) (end 134 93.875) (width 1.8) (layer "F.Cu") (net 1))
 (segment (start 153.85 84.46) (end 151.83 84.46) (width 1.8) (layer "F.Cu") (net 1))
 (segment (start 132.35 76.95) (end 133.75 75.55) (width 1.8) (layer "F.Cu") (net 1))
 (segment (start 150.3 85.99) (end 150.3 88.79) (width 1.8) (layer "F.Cu") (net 1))
 (segment (start 129.121321 81.5) (end 132.35 78.271321) (width 1.8) (layer "F.Cu") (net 1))
 (segment (start 133.75 73.55629) (end 133.75 73.55) (width 0.25) (layer "F.Cu") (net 1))
 (segment (start 140.95 94.9) (end 146.2125 94.9) (width 1.8) (layer "F.Cu") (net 1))
 (segment (start 137.1 73.3) (end 135.14 73.3) (width 1.8) (layer "F.Cu") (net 1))
 (segment (start 129.15 90.29) (end 132.735 93.875) (width 1.8) (layer "F.Cu") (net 1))
 (segment (start 135.14 73.3) (end 134 73.3) (width 1.8) (layer "F.Cu") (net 1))
 (segment (start 153.85 87) (end 152.14 87) (width 1.8) (layer "F.Cu") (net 1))
 (segment (start 140.079 78.9) (end 137.225 78.9) (width 1.8) (layer "F.Cu") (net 1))
 (segment (start 132.275 98.55) (end 134 96.825) (width 0.25) (layer "F.Cu") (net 10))
 (segment (start 132.275 99.6) (end 132.275 98.55) (width 0.25) (layer "F.Cu") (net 10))
 (segment (start 135 83.375) (end 135 79.625) (width 0.5) (layer "F.Cu") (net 9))
 (segment (start 135 79.625) (end 134.025 78.65) (width 0.5) (layer "F.Cu") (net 9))
 (segment (start 172.67 87.2) (end 169.93 84.46) (width 0.6) (layer "F.Cu") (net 15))
 (segment (start 173.2 87.2) (end 172.67 87.2) (width 0.6) (layer "F.Cu") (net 15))
 (segment (start 169.93 84.46) (end 166.63 84.46) (width 0.6) (layer "F.Cu") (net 15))
 (segment (start 166.63 87) (end 169.72 87) (width 0.6) (layer "F.Cu") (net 16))
 (segment (start 170.48 87.77) (end 171.81 89.1) (width 0.6) (layer "F.Cu") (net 16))
 (segment (start 170.48 87.76) (end 170.48 87.77) (width 0.6) (layer "F.Cu") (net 16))
 (segment (start 171.81 89.1) (end 173.2 89.1) (width 0.6) (layer "F.Cu") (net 16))
 (segment (start 173.45 89.35) (end 173.45 94.3) (width 0.6) (layer "F.Cu") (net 16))
 (segment (start 173.2 89.1) (end 173.45 89.35) (width 0.25) (layer "F.Cu") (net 16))
 (segment (start 166.63 87) (end 166.63 89.54) (width 0.25) (layer "F.Cu") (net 16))
 (segment (start 166.63 92.08) (end 166.63 89.54) (width 0.25) (layer "F.Cu") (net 16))
 (segment (start 169.72 87) (end 170.48 87.76) (width 0.6) (layer "F.Cu") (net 16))
 (segment (start 179.0375 75.05) (end 179 75.0875) (width 0.25) (layer "F.Cu") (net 14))
 (segment (start 175.1375 75.0875) (end 174.05 74) (width 0.25) (layer "F.Cu") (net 14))
 (segment (start 168.1 74) (end 167.8 74.3) (width 0.25) (layer "F.Cu") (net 14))
 (segment (start 174.05 74) (end 168.1 74) (width 0.25) (layer "F.Cu") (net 14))
 (segment (start 182.5 75.05) (end 179.0375 75.05) (width 0.25) (layer "F.Cu") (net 14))
 (segment (start 179 75.0875) (end 175.1375 75.0875) (width 0.25) (layer "F.Cu") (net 14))
 (segment (start 167.8 74.3) (end 166.63 74.3) (width 0.25) (layer "F.Cu") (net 14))
 (segment (start 177 78.9125) (end 175 78.9125) (width 0.8) (layer "F.Cu") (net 8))
 (segment (start 171.29 81.27) (end 171.57 81.55) (width 1.8) (layer "F.Cu") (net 8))
 (segment (start 174.5325 79.38) (end 175 78.9125) (width 1.8) (layer "F.Cu") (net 8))
 (segment (start 185.8 90.7) (end 183 93.5) (width 1.6) (layer "F.Cu") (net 8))
 (segment (start 166.63 79.38) (end 171.29 79.38) (width 1.8) (layer "F.Cu") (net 8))
 (segment (start 171.29 79.38) (end 174.5325 79.38) (width 1.8) (layer "F.Cu") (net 8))
 (segment (start 182.5 76.95) (end 179.0375 76.95) (width 0.8) (layer "F.Cu") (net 8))
 (segment (start 184.3 84.25) (end 185.8 85.75) (width 1.6) (layer "F.Cu") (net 8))
 (segment (start 179.0375 76.95) (end 179 76.9125) (width 0.25) (layer "F.Cu") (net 8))
 (segment (start 179 76.9125) (end 177 78.9125) (width 0.8) (layer "F.Cu") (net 8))
 (segment (start 175 91.75) (end 177.55 94.3) (width 1.6) (layer "F.Cu") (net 8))
 (segment (start 175 84.4) (end 175 91.75) (width 1.6) (layer "F.Cu") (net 8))
 (segment (start 181.7 84.25) (end 184.3 84.25) (width 1.6) (layer "F.Cu") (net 8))
 (segment (start 178.475 87.475) (end 181.7 84.25) (width 1.6) (layer "F.Cu") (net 8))
 (segment (start 177.55 87.925) (end 177.55 94.3) (width 1.6) (layer "F.Cu") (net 8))
 (segment (start 178 87.475) (end 177.55 87.925) (width 0.25) (layer "F.Cu") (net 8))
 (segment (start 171.29 79.38) (end 171.29 81.27) (width 1.8) (layer "F.Cu") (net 8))
 (segment (start 178 87.475) (end 178.475 87.475) (width 0.25) (layer "F.Cu") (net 8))
 (segment (start 185.8 85.75) (end 185.8 90.7) (width 1.6) (layer "F.Cu") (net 8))
 (via (at 171.57 81.55) (size 1.8) (drill 1.6) (layers "F.Cu" "B.Cu") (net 8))
 (via (at 175 84.4) (size 1.8) (drill 1.6) (layers "F.Cu" "B.Cu") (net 8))
 (segment (start 171.57 81.55) (end 173.29 81.55) (width 1.6) (layer "B.Cu") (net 8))
 (segment (start 173.29 81.55) (end 175 83.26) (width 1.6) (layer "B.Cu") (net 8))
 (segment (start 175 83.26) (end 175 84.4) (width 1.6) (layer "B.Cu") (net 8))
 (segment (start 166.63 81.92) (end 167.91 83.2) (width 0.25) (layer "F.Cu") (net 13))
 (segment (start 167.91 83.2) (end 175.1875 83.2) (width 0.25) (layer "F.Cu") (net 13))
 (segment (start 175.1875 83.2) (end 176.4375 81.95) (width 0.25) (layer "F.Cu") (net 13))
 (segment (start 150.2 73.19) (end 153.85 76.84) (width 0.25) (layer "F.Cu") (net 4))
 (segment (start 150.2 71) (end 150.2 73.19) (width 0.25) (layer "F.Cu") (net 4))
 (segment (start 137.1 71.4) (end 137.15 71.35) (width 0.25) (layer "F.Cu") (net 17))
 (segment (start 137.15 71.35) (end 141 71.35) (width 0.8) (layer "F.Cu") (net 17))
 (segment (start 129.25 73.6) (end 129.25 75) (width 0.8) (layer "F.Cu") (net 2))
 (segment (start 129.25 75) (end 130 75.75) (width 0.8) (layer "F.Cu") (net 2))
 (segment (start 131.85 73.55) (end 129.3 73.55) (width 0.8) (layer "F.Cu") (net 2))
 (segment (start 129.3 73.55) (end 129.25 73.6) (width 0.25) (layer "F.Cu") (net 2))
 (segment (start 140 97.75) (end 140.95 96.8) (width 0.25) (layer "F.Cu") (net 11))
 (segment (start 140 99.35) (end 140 97.75) (width 0.25) (layer "F.Cu") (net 11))
 (segment (start 153.85 79.38) (end 152.0675 79.38) (width 0.25) (layer "F.Cu") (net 5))
 (segment (start 152.0675 79.38) (end 145.9875 73.3) (width 0.25) (layer "F.Cu") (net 5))
 (segment (start 145.5875 99.35) (end 145.5875 97.425) (width 0.25) (layer "F.Cu") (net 6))
 (segment (start 153.85 81.92) (end 156.2 84.27) (width 0.25) (layer "F.Cu") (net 6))
 (segment (start 153.1875 96.7625) (end 146.25 96.7625) (width 0.25) (layer "F.Cu") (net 6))
 (segment (start 156.2 93.75) (end 153.1875 96.7625) (width 0.25) (layer "F.Cu") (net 6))
 (segment (start 145.5875 97.425) (end 146.25 96.7625) (width 0.25) (layer "F.Cu") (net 6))
 (segment (start 156.2 84.27) (end 156.2 93.75) (width 0.25) (layer "F.Cu") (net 6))
 (segment (start 175 77.0875) (end 174.7525 76.84) (width 0.25) (layer "F.Cu") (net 7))
 (segment (start 174.7525 76.84) (end 166.63 76.84) (width 0.25) (layer "F.Cu") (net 7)))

